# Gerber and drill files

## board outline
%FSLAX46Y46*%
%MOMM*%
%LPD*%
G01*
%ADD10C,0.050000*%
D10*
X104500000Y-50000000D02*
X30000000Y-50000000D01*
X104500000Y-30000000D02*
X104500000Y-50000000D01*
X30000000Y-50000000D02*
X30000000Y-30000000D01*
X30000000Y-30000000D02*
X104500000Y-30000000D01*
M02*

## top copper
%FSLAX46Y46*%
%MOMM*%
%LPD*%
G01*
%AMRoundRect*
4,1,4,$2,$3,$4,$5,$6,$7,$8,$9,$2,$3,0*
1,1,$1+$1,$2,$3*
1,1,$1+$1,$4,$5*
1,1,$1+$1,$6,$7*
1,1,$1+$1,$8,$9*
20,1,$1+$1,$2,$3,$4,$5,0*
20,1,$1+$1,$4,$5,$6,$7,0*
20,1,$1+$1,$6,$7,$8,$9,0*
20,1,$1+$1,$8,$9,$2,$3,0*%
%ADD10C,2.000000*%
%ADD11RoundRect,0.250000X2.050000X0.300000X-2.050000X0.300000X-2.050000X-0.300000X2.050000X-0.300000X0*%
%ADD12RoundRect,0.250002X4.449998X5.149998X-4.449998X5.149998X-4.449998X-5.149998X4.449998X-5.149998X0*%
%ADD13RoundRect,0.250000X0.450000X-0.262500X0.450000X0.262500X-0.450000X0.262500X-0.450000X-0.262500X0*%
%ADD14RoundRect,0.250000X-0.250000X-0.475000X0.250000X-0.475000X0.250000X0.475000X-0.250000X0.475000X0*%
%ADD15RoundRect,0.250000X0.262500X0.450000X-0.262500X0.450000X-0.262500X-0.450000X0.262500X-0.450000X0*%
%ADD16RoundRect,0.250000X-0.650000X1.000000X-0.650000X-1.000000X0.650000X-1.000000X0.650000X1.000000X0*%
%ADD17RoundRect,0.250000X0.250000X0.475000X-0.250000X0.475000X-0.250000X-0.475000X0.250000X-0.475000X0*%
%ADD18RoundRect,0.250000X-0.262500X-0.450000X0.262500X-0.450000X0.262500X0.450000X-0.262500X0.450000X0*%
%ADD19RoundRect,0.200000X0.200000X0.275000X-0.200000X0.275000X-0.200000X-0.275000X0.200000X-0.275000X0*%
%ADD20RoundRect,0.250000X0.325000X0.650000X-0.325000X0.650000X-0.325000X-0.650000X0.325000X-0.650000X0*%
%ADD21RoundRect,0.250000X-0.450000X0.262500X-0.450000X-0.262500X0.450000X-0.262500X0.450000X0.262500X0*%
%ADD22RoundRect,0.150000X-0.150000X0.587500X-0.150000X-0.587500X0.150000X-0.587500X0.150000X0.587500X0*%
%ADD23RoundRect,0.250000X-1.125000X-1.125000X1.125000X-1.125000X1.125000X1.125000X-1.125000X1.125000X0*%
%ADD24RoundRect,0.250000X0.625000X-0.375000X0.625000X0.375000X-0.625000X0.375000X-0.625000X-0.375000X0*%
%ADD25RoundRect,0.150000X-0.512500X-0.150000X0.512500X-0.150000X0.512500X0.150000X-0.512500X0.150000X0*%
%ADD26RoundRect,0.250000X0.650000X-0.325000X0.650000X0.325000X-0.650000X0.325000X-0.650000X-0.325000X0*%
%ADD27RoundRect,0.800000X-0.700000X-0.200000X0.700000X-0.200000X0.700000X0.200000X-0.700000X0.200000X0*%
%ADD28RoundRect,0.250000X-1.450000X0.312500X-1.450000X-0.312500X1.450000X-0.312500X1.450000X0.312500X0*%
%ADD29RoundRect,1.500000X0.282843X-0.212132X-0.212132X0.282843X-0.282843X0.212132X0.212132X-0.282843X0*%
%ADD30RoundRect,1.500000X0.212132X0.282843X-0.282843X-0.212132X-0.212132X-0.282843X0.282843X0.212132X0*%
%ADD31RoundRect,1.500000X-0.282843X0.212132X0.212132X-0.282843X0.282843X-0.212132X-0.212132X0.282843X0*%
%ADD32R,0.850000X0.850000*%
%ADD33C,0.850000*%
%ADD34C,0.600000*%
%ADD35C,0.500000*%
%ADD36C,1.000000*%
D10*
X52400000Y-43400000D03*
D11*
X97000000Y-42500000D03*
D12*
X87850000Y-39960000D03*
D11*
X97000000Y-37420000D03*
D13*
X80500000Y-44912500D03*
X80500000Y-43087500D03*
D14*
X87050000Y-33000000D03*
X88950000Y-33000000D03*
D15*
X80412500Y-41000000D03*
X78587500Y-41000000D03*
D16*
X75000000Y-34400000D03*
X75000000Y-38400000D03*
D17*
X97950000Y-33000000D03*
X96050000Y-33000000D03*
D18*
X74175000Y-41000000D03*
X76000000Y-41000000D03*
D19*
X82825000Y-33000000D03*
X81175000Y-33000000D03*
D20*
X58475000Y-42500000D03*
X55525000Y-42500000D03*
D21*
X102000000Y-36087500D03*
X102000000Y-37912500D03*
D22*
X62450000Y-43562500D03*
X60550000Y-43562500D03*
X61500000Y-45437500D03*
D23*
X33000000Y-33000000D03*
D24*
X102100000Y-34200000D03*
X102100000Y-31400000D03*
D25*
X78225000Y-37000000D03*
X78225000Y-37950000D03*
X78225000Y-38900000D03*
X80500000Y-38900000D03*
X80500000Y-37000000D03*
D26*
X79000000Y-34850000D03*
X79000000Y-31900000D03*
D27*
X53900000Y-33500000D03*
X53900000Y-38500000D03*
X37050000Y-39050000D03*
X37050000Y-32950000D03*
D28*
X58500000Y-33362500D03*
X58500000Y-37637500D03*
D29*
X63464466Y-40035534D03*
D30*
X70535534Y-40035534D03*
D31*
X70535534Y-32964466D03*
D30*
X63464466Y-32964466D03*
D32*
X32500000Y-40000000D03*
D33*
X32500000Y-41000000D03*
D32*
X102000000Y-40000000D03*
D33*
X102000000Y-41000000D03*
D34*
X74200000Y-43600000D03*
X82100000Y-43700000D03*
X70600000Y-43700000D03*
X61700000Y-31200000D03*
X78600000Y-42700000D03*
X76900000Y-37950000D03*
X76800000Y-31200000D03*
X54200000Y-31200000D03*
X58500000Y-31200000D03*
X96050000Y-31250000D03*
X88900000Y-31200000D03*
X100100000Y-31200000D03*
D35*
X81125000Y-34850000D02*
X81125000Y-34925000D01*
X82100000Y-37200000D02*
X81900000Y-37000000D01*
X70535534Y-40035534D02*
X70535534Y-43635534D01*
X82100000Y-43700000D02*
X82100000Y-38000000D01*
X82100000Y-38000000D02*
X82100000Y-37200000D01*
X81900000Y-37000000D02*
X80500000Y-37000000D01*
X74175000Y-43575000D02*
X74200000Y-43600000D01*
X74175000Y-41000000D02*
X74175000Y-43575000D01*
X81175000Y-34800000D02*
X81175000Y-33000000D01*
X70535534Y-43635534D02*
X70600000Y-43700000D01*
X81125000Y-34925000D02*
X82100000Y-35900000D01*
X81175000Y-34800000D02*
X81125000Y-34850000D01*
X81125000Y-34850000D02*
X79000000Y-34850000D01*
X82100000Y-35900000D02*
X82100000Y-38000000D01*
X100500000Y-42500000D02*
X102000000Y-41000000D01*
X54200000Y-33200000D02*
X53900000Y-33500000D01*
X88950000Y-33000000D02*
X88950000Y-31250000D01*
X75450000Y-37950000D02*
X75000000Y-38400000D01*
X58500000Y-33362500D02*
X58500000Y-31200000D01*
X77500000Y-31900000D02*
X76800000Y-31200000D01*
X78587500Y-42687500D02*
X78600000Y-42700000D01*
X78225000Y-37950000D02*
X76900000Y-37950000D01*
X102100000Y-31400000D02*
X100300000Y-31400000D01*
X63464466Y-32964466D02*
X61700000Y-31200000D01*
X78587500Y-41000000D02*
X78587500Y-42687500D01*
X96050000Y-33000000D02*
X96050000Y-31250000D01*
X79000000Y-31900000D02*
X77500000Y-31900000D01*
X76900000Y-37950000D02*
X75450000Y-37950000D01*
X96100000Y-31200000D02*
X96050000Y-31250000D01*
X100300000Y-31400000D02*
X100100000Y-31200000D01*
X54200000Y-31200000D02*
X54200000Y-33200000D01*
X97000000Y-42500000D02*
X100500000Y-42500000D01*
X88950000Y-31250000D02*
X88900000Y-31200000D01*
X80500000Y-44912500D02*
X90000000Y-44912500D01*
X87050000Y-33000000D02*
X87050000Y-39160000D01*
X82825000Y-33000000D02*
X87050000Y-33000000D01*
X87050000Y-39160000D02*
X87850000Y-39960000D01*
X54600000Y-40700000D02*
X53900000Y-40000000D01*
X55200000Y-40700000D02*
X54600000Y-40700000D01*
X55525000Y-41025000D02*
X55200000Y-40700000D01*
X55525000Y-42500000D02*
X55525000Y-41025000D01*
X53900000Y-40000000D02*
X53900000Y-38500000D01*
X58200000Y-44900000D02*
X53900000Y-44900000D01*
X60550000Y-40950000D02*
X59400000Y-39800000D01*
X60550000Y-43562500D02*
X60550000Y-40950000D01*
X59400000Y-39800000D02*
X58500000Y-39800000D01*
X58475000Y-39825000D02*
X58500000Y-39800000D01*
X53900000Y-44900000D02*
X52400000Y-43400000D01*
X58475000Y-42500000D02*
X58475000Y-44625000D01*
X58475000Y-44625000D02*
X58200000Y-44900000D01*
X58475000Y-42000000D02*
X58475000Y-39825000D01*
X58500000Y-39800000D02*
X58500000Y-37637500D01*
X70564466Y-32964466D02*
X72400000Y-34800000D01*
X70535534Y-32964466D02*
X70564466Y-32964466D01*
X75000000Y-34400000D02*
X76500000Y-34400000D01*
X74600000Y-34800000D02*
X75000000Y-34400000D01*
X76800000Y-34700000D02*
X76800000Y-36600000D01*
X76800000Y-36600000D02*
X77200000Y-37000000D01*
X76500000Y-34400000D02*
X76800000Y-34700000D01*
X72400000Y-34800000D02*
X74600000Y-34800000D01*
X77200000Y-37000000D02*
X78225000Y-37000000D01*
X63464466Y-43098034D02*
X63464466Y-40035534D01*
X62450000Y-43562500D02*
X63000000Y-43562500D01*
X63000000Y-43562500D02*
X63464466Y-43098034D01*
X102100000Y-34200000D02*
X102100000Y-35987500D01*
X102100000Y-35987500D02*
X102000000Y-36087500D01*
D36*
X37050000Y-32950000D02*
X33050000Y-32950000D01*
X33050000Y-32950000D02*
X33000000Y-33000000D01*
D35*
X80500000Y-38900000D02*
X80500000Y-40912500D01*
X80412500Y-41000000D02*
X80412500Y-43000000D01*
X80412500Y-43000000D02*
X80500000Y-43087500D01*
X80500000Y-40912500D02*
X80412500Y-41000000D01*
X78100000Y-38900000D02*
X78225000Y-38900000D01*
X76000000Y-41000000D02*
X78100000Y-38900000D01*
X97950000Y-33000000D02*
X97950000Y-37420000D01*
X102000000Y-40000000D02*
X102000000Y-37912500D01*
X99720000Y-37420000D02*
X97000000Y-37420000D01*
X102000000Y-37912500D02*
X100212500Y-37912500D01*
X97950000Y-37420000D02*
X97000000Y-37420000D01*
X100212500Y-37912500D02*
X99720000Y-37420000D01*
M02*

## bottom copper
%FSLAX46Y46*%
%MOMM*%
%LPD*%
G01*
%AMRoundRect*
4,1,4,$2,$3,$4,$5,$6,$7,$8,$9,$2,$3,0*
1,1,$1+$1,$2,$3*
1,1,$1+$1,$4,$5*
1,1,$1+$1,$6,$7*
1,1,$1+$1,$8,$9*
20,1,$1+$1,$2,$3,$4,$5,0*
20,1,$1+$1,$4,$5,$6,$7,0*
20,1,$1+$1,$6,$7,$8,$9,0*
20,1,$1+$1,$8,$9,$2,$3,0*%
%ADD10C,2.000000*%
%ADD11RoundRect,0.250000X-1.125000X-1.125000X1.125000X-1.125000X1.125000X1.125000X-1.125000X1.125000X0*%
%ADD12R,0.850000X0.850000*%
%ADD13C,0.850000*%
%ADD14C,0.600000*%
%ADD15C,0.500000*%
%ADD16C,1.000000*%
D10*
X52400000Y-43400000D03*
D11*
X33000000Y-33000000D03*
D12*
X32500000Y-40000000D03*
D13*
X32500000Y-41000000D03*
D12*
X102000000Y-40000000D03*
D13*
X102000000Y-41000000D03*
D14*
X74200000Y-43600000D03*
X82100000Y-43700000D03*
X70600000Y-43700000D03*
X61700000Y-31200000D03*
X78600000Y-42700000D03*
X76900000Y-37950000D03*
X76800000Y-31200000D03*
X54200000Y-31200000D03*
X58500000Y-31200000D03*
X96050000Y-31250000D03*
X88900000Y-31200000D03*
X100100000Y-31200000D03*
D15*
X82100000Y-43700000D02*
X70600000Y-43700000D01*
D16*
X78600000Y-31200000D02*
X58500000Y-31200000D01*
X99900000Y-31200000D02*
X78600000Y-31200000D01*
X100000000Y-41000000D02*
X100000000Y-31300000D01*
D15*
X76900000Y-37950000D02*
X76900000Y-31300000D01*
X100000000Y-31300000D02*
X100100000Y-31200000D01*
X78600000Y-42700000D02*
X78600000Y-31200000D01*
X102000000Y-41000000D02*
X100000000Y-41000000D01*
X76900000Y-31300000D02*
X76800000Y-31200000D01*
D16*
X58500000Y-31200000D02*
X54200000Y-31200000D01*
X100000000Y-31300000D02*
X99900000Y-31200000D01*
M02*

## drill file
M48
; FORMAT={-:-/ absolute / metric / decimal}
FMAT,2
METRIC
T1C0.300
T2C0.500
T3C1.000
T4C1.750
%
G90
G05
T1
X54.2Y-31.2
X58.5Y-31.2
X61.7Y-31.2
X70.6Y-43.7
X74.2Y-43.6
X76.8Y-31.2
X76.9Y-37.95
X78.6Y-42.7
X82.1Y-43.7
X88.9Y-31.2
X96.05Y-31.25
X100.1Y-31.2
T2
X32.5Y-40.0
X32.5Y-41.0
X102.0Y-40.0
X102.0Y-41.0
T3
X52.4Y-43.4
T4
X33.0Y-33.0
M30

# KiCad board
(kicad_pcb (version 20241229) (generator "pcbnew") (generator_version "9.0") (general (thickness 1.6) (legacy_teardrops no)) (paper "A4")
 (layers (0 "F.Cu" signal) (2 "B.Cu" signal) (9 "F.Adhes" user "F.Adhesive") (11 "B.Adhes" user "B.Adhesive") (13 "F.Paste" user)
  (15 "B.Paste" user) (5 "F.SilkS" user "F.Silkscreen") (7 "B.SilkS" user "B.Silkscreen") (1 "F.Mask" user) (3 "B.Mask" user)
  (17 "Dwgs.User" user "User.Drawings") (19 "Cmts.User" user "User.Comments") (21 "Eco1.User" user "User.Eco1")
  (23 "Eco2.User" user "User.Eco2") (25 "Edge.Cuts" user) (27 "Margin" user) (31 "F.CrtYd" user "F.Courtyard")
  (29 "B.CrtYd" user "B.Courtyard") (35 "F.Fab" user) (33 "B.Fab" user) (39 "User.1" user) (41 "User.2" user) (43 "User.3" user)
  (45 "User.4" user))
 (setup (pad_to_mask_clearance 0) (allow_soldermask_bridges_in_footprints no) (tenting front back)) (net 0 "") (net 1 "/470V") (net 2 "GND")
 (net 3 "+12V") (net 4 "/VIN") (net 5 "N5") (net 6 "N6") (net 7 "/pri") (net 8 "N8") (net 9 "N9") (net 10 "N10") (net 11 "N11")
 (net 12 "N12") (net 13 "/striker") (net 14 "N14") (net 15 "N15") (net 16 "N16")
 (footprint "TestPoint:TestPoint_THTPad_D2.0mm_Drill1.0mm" (layer "F.Cu") (at 52.4 43.4)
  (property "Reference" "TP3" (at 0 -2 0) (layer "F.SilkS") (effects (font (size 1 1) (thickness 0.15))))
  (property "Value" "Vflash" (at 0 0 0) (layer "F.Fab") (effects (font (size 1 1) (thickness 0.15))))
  (pad "1" thru_hole circle (at 0 0) (size 2 2) (drill 1) (layers "*.Cu" "*.Mask") (remove_unused_layers no) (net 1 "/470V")))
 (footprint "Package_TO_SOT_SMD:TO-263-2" (layer "F.Cu") (at 89.35 39.96 180)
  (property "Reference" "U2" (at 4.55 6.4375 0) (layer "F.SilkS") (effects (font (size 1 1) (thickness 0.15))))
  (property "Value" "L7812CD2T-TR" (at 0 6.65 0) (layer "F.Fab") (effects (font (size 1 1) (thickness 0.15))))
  (pad "" smd roundrect (at -0.925 -2.775 180) (size 4.55 5.25) (layers "F.Paste") (roundrect_rratio 0.054945))
  (pad "" smd roundrect (at -0.925 2.775 180) (size 4.55 5.25) (layers "F.Paste") (roundrect_rratio 0.054945))
  (pad "" smd roundrect (at 3.925 -2.775 180) (size 4.55 5.25) (layers "F.Paste") (roundrect_rratio 0.054945))
  (pad "" smd roundrect (at 3.925 2.775 180) (size 4.55 5.25) (layers "F.Paste") (roundrect_rratio 0.054945))
  (pad "1" smd roundrect (at -7.65 -2.54 180) (size 4.6 1.1) (layers "F.Cu" "F.Mask" "F.Paste") (roundrect_rratio 0.227273) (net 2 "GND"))
  (pad "2" smd roundrect (at 1.5 0 180) (size 9.4 10.8) (layers "F.Cu" "F.Mask") (roundrect_rratio 0.026596) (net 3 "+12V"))
  (pad "3" smd roundrect (at -7.65 2.54 180) (size 4.6 1.1) (layers "F.Cu" "F.Mask" "F.Paste") (roundrect_rratio 0.227273) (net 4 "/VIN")))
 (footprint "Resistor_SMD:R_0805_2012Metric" (layer "F.Cu") (at 80.5 44 90)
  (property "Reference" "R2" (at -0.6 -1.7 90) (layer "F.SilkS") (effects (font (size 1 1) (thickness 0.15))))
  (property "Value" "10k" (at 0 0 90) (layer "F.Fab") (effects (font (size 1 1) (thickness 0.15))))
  (pad "1" smd roundrect (at -0.9125 0 90) (size 1.025 1.4) (layers "F.Cu" "F.Mask" "F.Paste") (roundrect_rratio 0.243902) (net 3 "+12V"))
  (pad "2" smd roundrect (at 0.9125 0 90) (size 1.025 1.4) (layers "F.Cu" "F.Mask" "F.Paste") (roundrect_rratio 0.243902) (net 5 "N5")))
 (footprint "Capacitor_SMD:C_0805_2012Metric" (layer "F.Cu") (at 88 33)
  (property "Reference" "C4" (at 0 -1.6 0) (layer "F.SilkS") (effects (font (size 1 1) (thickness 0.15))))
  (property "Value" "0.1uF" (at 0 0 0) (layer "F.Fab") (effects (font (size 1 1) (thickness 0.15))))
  (pad "1" smd roundrect (at -0.95 0) (size 1 1.45) (layers "F.Cu" "F.Mask" "F.Paste") (roundrect_rratio 0.25) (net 3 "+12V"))
  (pad "2" smd roundrect (at 0.95 0) (size 1 1.45) (layers "F.Cu" "F.Mask" "F.Paste") (roundrect_rratio 0.25) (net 2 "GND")))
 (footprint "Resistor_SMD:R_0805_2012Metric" (layer "F.Cu") (at 79.5 41 180)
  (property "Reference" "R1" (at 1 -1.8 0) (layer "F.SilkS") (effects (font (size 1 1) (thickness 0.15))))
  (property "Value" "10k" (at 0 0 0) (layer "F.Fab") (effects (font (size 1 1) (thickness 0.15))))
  (pad "1" smd roundrect (at -0.9125 0 180) (size 1.025 1.4) (layers "F.Cu" "F.Mask" "F.Paste") (roundrect_rratio 0.243902) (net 5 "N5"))
  (pad "2" smd roundrect (at 0.9125 0 180) (size 1.025 1.4) (layers "F.Cu" "F.Mask" "F.Paste") (roundrect_rratio 0.243902) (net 2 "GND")))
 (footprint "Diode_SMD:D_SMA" (layer "F.Cu") (at 75 36.4 -90)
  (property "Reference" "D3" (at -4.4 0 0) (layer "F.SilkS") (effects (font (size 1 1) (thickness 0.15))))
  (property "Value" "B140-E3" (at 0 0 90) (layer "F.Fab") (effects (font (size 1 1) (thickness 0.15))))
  (pad "1" smd roundrect (at -2 0 270) (size 2.5 1.8) (layers "F.Cu" "F.Mask" "F.Paste") (roundrect_rratio 0.1388888889) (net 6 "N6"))
  (pad "2" smd roundrect (at 2 0 270) (size 2.5 1.8) (layers "F.Cu" "F.Mask" "F.Paste") (roundrect_rratio 0.1388888889) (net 2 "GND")))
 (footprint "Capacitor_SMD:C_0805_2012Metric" (layer "F.Cu") (at 97 33 180)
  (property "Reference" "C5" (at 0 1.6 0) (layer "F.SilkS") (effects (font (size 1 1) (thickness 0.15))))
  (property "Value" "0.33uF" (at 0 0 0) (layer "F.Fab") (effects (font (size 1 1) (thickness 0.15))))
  (pad "1" smd roundrect (at -0.95 0 180) (size 1 1.45) (layers "F.Cu" "F.Mask" "F.Paste") (roundrect_rratio 0.25) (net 4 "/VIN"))
  (pad "2" smd roundrect (at 0.95 0 180) (size 1 1.45) (layers "F.Cu" "F.Mask" "F.Paste") (roundrect_rratio 0.25) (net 2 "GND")))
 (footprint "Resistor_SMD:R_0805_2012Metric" (layer "F.Cu") (at 75.0875 41)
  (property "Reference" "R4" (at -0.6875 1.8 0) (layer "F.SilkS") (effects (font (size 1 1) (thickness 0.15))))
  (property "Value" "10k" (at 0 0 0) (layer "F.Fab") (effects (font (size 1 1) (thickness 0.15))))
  (pad "1" smd roundrect (at -0.9125 0) (size 1.025 1.4) (layers "F.Cu" "F.Mask" "F.Paste") (roundrect_rratio 0.243902) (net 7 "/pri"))
  (pad "2" smd roundrect (at 0.9125 0) (size 1.025 1.4) (layers "F.Cu" "F.Mask" "F.Paste") (roundrect_rratio 0.243902) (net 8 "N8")))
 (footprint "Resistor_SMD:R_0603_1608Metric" (layer "F.Cu") (at 82 33 180)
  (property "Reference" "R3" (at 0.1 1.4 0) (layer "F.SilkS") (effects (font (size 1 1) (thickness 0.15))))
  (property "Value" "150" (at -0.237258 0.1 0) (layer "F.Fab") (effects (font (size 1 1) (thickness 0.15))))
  (pad "1" smd roundrect (at -0.825 0 180) (size 0.8 0.95) (layers "F.Cu" "F.Mask" "F.Paste") (roundrect_rratio 0.25) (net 3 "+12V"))
  (pad "2" smd roundrect (at 0.825 0 180) (size 0.8 0.95) (layers "F.Cu" "F.Mask" "F.Paste") (roundrect_rratio 0.25) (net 7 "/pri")))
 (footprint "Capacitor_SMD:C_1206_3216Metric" (layer "F.Cu") (at 57 42.5 180)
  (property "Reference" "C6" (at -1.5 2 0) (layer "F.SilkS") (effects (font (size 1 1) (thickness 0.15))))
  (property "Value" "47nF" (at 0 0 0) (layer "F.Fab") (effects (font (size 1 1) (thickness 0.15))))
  (pad "1" smd roundrect (at -1.475 0 180) (size 1.15 1.8) (layers "F.Cu" "F.Mask" "F.Paste") (roundrect_rratio 0.217391) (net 1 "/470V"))
  (pad "2" smd roundrect (at 1.475 0 180) (size 1.15 1.8) (layers "F.Cu" "F.Mask" "F.Paste") (roundrect_rratio 0.217391) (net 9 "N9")))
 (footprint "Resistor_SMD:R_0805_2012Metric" (layer "F.Cu") (at 102 37 -90)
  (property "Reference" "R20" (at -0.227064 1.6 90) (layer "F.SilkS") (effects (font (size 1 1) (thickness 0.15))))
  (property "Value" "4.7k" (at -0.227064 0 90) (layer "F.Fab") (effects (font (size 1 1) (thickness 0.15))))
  (pad "1" smd roundrect (at -0.9125 0 270) (size 1.025 1.4) (layers "F.Cu" "F.Mask" "F.Paste") (roundrect_rratio 0.243902) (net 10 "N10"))
  (pad "2" smd roundrect (at 0.9125 0 270) (size 1.025 1.4) (layers "F.Cu" "F.Mask" "F.Paste") (roundrect_rratio 0.243902) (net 4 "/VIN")))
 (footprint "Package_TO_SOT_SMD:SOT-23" (layer "F.Cu") (at 61.5 44.5 -90)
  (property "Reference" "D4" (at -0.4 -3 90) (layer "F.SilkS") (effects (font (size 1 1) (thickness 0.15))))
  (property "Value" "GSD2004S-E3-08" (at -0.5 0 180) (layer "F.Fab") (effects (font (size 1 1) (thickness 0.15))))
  (pad "1" smd roundrect (at -0.9375 -0.95 270) (size 1.475 0.6) (layers "F.Cu" "F.Mask" "F.Paste") (roundrect_rratio 0.25) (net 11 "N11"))
  (pad "2" smd roundrect (at -0.9375 0.95 270) (size 1.475 0.6) (layers "F.Cu" "F.Mask" "F.Paste") (roundrect_rratio 0.25) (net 1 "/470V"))
  (pad "3" smd roundrect (at 0.9375 0 270) (size 1.475 0.6) (layers "F.Cu" "F.Mask" "F.Paste") (roundrect_rratio 0.25) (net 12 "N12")))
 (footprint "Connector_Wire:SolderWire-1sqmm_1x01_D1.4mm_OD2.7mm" (layer "F.Cu") (at 33 33)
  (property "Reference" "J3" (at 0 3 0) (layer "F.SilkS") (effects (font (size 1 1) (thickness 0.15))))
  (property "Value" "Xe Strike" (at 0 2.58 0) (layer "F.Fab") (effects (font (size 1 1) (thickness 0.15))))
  (pad "1" thru_hole roundrect (at 0 0) (size 2.75 2.75) (drill 1.75) (layers "*.Cu" "*.Mask") (remove_unused_layers no)
   (roundrect_rratio 0.090909) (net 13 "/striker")))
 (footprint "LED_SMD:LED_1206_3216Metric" (layer "F.Cu") (at 102.1 32.8 90)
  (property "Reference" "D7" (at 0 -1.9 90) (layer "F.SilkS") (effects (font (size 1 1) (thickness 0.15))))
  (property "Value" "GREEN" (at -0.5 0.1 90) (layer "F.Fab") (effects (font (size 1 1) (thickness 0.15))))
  (pad "1" smd roundrect (at -1.4 0 90) (size 1.25 1.75) (layers "F.Cu" "F.Mask" "F.Paste") (roundrect_rratio 0.2) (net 10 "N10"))
  (pad "2" smd roundrect (at 1.4 0 90) (size 1.25 1.75) (layers "F.Cu" "F.Mask" "F.Paste") (roundrect_rratio 0.2) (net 2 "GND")))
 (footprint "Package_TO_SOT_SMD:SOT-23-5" (layer "F.Cu") (at 79.3625 37.95)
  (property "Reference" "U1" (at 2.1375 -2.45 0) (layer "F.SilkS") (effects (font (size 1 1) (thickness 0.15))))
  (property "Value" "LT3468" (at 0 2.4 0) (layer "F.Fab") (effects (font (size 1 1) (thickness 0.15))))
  (pad "1" smd roundrect (at -1.1375 -0.95) (size 1.325 0.6) (layers "F.Cu" "F.Mask" "F.Paste") (roundrect_rratio 0.25) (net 6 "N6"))
  (pad "2" smd roundrect (at -1.1375 0) (size 1.325 0.6) (layers "F.Cu" "F.Mask" "F.Paste") (roundrect_rratio 0.25) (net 2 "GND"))
  (pad "3" smd roundrect (at -1.1375 0.95) (size 1.325 0.6) (layers "F.Cu" "F.Mask" "F.Paste") (roundrect_rratio 0.25) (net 8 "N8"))
  (pad "4" smd roundrect (at 1.1375 0.95) (size 1.325 0.6) (layers "F.Cu" "F.Mask" "F.Paste") (roundrect_rratio 0.25) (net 5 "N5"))
  (pad "5" smd roundrect (at 1.1375 -0.95) (size 1.325 0.6) (layers "F.Cu" "F.Mask" "F.Paste") (roundrect_rratio 0.25) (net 7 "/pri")))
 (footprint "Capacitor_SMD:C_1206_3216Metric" (layer "F.Cu") (at 79 33.375 90)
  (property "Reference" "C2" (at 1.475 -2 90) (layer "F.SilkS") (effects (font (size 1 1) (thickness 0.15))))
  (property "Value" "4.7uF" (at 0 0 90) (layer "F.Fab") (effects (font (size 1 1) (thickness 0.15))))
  (pad "1" smd roundrect (at -1.475 0 90) (size 1.15 1.8) (layers "F.Cu" "F.Mask" "F.Paste") (roundrect_rratio 0.217391) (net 7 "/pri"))
  (pad "2" smd roundrect (at 1.475 0 90) (size 1.15 1.8) (layers "F.Cu" "F.Mask" "F.Paste") (roundrect_rratio 0.217391) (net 2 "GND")))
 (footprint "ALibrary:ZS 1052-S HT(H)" (layer "F.Cu") (at 45.5 36 180)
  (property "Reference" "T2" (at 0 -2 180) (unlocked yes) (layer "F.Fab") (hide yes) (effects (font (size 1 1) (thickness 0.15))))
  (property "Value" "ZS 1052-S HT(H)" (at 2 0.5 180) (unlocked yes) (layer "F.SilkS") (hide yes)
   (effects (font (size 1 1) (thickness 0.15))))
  (pad "1" smd roundrect (at -8.4 2.5) (size 3 2) (layers "F.Cu" "F.Mask" "F.Paste") (roundrect_rratio 0.4) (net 2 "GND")
   (thermal_bridge_angle 45))
  (pad "2" smd roundrect (at -8.4 -2.5) (size 3 2) (layers "F.Cu" "F.Mask" "F.Paste") (roundrect_rratio 0.4) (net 9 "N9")
   (thermal_bridge_angle 45))
  (pad "3" smd roundrect (at 8.45 -3.05) (size 3 2) (layers "F.Cu" "F.Mask" "F.Paste") (roundrect_rratio 0.4) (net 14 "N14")
   (thermal_bridge_angle 45))
  (pad "4" smd roundrect (at 8.45 3.05) (size 3 2) (layers "F.Cu" "F.Mask" "F.Paste") (roundrect_rratio 0.4) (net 13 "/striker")
   (thermal_bridge_angle 45)))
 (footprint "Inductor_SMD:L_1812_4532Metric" (layer "F.Cu") (at 58.5 35.5 -90)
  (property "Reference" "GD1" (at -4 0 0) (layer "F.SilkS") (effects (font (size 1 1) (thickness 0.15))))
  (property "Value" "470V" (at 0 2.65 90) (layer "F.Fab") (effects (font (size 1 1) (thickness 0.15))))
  (pad "1" smd roundrect (at -2.1375 0 270) (size 1.125 3.4) (layers "F.Cu" "F.Mask" "F.Paste") (roundrect_rratio 0.222222) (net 2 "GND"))
  (pad "2" smd roundrect (at 2.1375 0 270) (size 1.125 3.4) (layers "F.Cu" "F.Mask" "F.Paste") (roundrect_rratio 0.222222) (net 1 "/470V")))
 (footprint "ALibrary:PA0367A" (layer "F.Cu") (at 67 36.5 135)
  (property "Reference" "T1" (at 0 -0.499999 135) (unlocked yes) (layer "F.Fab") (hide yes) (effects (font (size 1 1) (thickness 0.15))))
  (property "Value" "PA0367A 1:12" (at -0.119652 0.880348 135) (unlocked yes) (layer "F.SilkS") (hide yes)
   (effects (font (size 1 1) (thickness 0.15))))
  (pad "1" smd roundrect (at 0 -5 135) (size 3.7 3.1) (layers "F.Cu" "F.Mask" "F.Paste") (roundrect_rratio 0.4838709677) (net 11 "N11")
   (thermal_bridge_angle 45))
  (pad "2" smd roundrect (at -5 0 225) (size 3.7 3.1) (layers "F.Cu" "F.Mask" "F.Paste") (roundrect_rratio 0.4838709677) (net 7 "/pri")
   (thermal_bridge_angle 45))
  (pad "3" smd roundrect (at 0 5 315) (size 3.7 3.1) (layers "F.Cu" "F.Mask" "F.Paste") (roundrect_rratio 0.4838709677) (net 6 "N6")
   (thermal_bridge_angle 45))
  (pad "4" smd roundrect (at 5 0 225) (size 3.7 3.1) (layers "F.Cu" "F.Mask" "F.Paste") (roundrect_rratio 0.4838709677) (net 2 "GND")
   (thermal_bridge_angle 45)))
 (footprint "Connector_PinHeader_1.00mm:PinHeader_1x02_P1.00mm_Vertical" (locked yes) (layer "B.Cu") (at 32.5 40 180)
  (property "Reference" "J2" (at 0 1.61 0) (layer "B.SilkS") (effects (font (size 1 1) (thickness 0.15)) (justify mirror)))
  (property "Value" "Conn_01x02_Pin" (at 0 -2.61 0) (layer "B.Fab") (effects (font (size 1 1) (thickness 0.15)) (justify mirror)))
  (pad "1" thru_hole rect (at 0 0 180) (size 0.85 0.85) (drill 0.5) (layers "*.Cu" "*.Mask") (remove_unused_layers no) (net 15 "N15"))
  (pad "2" thru_hole circle (at 0 -1 180) (size 0.85 0.85) (drill 0.5) (layers "*.Cu" "*.Mask") (remove_unused_layers no) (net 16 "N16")))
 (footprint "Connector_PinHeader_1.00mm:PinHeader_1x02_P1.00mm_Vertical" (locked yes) (layer "B.Cu") (at 102 40 180)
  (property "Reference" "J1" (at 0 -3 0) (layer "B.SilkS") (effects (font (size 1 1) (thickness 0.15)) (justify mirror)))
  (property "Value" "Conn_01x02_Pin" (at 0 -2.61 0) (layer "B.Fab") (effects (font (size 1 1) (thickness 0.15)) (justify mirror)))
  (pad "1" thru_hole rect (at 0 0 180) (size 0.85 0.85) (drill 0.5) (layers "*.Cu" "*.Mask") (remove_unused_layers no) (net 4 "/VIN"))
  (pad "2" thru_hole circle (at 0 -1 180) (size 0.85 0.85) (drill 0.5) (layers "*.Cu" "*.Mask") (remove_unused_layers no) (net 2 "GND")))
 (gr_line (start 104.5 50) (end 30 50) (stroke (width 0.05) (type default)) (layer "Edge.Cuts"))
 (gr_line (start 104.5 30) (end 104.5 50) (stroke (width 0.05) (type default)) (layer "Edge.Cuts"))
 (gr_line (start 30 50) (end 30 30) (stroke (width 0.05) (type default)) (layer "Edge.Cuts"))
 (gr_line (start 30 30) (end 104.5 30) (stroke (width 0.05) (type default)) (layer "Edge.Cuts"))
 (segment (start 81.125 34.85) (end 81.125 34.925) (width 0.5) (layer "F.Cu") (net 7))
 (segment (start 82.1 37.2) (end 81.9 37) (width 0.5) (layer "F.Cu") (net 7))
 (segment (start 70.535534 40.035534) (end 70.535534 43.635534) (width 0.5) (layer "F.Cu") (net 7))
 (segment (start 82.1 43.7) (end 82.1 38) (width 0.5) (layer "F.Cu") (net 7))
 (segment (start 82.1 38) (end 82.1 37.2) (width 0.5) (layer "F.Cu") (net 7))
 (segment (start 81.9 37) (end 80.5 37) (width 0.5) (layer "F.Cu") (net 7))
 (segment (start 74.175 43.575) (end 74.2 43.6) (width 0.5) (layer "F.Cu") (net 7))
 (segment (start 74.175 41) (end 74.175 43.575) (width 0.5) (layer "F.Cu") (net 7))
 (segment (start 81.175 34.8) (end 81.175 33) (width 0.5) (layer "F.Cu") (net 7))
 (segment (start 70.535534 43.635534) (end 70.6 43.7) (width 0.5) (layer "F.Cu") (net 7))
 (segment (start 81.125 34.925) (end 82.1 35.9) (width 0.5) (layer "F.Cu") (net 7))
 (segment (start 81.175 34.8) (end 81.125 34.85) (width 0.5) (layer "F.Cu") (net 7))
 (segment (start 81.125 34.85) (end 79 34.85) (width 0.5) (layer "F.Cu") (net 7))
 (segment (start 82.1 35.9) (end 82.1 38) (width 0.5) (layer "F.Cu") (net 7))
 (via (at 74.2 43.6) (size 0.6) (drill 0.3) (layers "F.Cu" "B.Cu") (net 7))
 (via (at 82.1 43.7) (size 0.6) (drill 0.3) (layers "F.Cu" "B.Cu") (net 7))
 (via (at 70.6 43.7) (size 0.6) (drill 0.3) (layers "F.Cu" "B.Cu") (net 7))
 (segment (start 82.1 43.7) (end 70.6 43.7) (width 0.5) (layer "B.Cu") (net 7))
 (segment (start 100.5 42.5) (end 102 41) (width 0.5) (layer "F.Cu") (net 2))
 (segment (start 54.2 33.2) (end 53.9 33.5) (width 0.5) (layer "F.Cu") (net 2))
 (segment (start 88.95 33) (end 88.95 31.25) (width 0.5) (layer "F.Cu") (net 2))
 (segment (start 75.45 37.95) (end 75 38.4) (width 0.5) (layer "F.Cu") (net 2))
 (segment (start 58.5 33.3625) (end 58.5 31.2) (width 0.5) (layer "F.Cu") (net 2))
 (segment (start 77.5 31.9) (end 76.8 31.2) (width 0.5) (layer "F.Cu") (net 2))
 (segment (start 78.5875 42.6875) (end 78.6 42.7) (width 0.5) (layer "F.Cu") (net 2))
 (segment (start 78.225 37.95) (end 76.9 37.95) (width 0.5) (layer "F.Cu") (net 2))
 (segment (start 102.1 31.4) (end 100.3 31.4) (width 0.5) (layer "F.Cu") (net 2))
 (segment (start 63.464466 32.964466) (end 61.7 31.2) (width 0.5) (layer "F.Cu") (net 2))
 (segment (start 78.5875 41) (end 78.5875 42.6875) (width 0.5) (layer "F.Cu") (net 2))
 (segment (start 96.05 33) (end 96.05 31.25) (width 0.5) (layer "F.Cu") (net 2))
 (segment (start 79 31.9) (end 77.5 31.9) (width 0.5) (layer "F.Cu") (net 2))
 (segment (start 76.9 37.95) (end 75.45 37.95) (width 0.5) (layer "F.Cu") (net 2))
 (segment (start 96.1 31.2) (end 96.05 31.25) (width 0.5) (layer "F.Cu") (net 2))
 (segment (start 100.3 31.4) (end 100.1 31.2) (width 0.5) (layer "F.Cu") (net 2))
 (segment (start 54.2 31.2) (end 54.2 33.2) (width 0.5) (layer "F.Cu") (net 2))
 (segment (start 97 42.5) (end 100.5 42.5) (width 0.5) (layer "F.Cu") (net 2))
 (segment (start 88.95 31.25) (end 88.9 31.2) (width 0.5) (layer "F.Cu") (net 2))
 (via (at 61.7 31.2) (size 0.6) (drill 0.3) (layers "F.Cu" "B.Cu") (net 2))
 (via (at 78.6 42.7) (size 0.6) (drill 0.3) (layers "F.Cu" "B.Cu") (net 2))
 (via (at 76.9 37.95) (size 0.6) (drill 0.3) (layers "F.Cu" "B.Cu") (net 2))
 (via (at 76.8 31.2) (size 0.6) (drill 0.3) (layers "F.Cu" "B.Cu") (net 2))
 (via (at 54.2 31.2) (size 0.6) (drill 0.3) (layers "F.Cu" "B.Cu") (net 2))
 (via (at 58.5 31.2) (size 0.6) (drill 0.3) (layers "F.Cu" "B.Cu") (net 2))
 (via (at 96.05 31.25) (size 0.6) (drill 0.3) (layers "F.Cu" "B.Cu") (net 2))
 (via (at 88.9 31.2) (size 0.6) (drill 0.3) (layers "F.Cu" "B.Cu") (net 2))
 (via (at 100.1 31.2) (size 0.6) (drill 0.3) (layers "F.Cu" "B.Cu") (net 2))
 (segment (start 78.6 31.2) (end 58.5 31.2) (width 1) (layer "B.Cu") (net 2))
 (segment (start 99.9 31.2) (end 78.6 31.2) (width 1) (layer "B.Cu") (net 2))
 (segment (start 100 41) (end 100 31.3) (width 1) (layer "B.Cu") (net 2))
 (segment (start 76.9 37.95) (end 76.9 31.3) (width 0.5) (layer "B.Cu") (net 2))
 (segment (start 100 31.3) (end 100.1 31.2) (width 0.5) (layer "B.Cu") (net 2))
 (segment (start 78.6 42.7) (end 78.6 31.2) (width 0.5) (layer "B.Cu") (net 2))
 (segment (start 102 41) (end 100 41) (width 0.5) (layer "B.Cu") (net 2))
 (segment (start 76.9 31.3) (end 76.8 31.2) (width 0.5) (layer "B.Cu") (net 2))
 (segment (start 58.5 31.2) (end 54.2 31.2) (width 1) (layer "B.Cu") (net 2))
 (segment (start 100 31.3) (end 99.9 31.2) (width 1) (layer "B.Cu") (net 2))
 (segment (start 80.5 44.9125) (end 90 44.9125) (width 0.5) (layer "F.Cu") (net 3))
 (segment (start 87.05 33) (end 87.05 39.16) (width 0.5) (layer "F.Cu") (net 3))
 (segment (start 82.825 33) (end 87.05 33) (width 0.5) (layer "F.Cu") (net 3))
 (segment (start 87.05 39.16) (end 87.85 39.96) (width 0.5) (layer "F.Cu") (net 3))
 (segment (start 54.6 40.7) (end 53.9 40) (width 0.5) (layer "F.Cu") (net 9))
 (segment (start 55.2 40.7) (end 54.6 40.7) (width 0.5) (layer "F.Cu") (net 9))
 (segment (start 55.525 41.025) (end 55.2 40.7) (width 0.5) (layer "F.Cu") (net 9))
 (segment (start 55.525 42.5) (end 55.525 41.025) (width 0.5) (layer "F.Cu") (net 9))
 (segment (start 53.9 40) (end 53.9 38.5) (width 0.5) (layer "F.Cu") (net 9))
 (segment (start 58.2 44.9) (end 53.9 44.9) (width 0.5) (layer "F.Cu") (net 1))
 (segment (start 60.55 40.95) (end 59.4 39.8) (width 0.5) (layer "F.Cu") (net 1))
 (segment (start 60.55 43.5625) (end 60.55 40.95) (width 0.5) (layer "F.Cu") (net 1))
 (segment (start 59.4 39.8) (end 58.5 39.8) (width 0.5) (layer "F.Cu") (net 1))
 (segment (start 58.475 39.825) (end 58.5 39.8) (width 0.5) (layer "F.Cu") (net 1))
 (segment (start 53.9 44.9) (end 52.4 43.4) (width 0.5) (layer "F.Cu") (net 1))
 (segment (start 58.475 42.5) (end 58.475 44.625) (width 0.5) (layer "F.Cu") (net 1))
 (segment (start 58.475 44.625) (end 58.2 44.9) (width 0.5) (layer "F.Cu") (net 1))
 (segment (start 58.475 42) (end 58.475 39.825) (width 0.5) (layer "F.Cu") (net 1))
 (segment (start 58.5 39.8) (end 58.5 37.6375) (width 0.5) (layer "F.Cu") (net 1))
 (segment (start 70.564466 32.964466) (end 72.4 34.8) (width 0.5) (layer "F.Cu") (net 6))
 (segment (start 70.535534 32.964466) (end 70.564466 32.964466) (width 0.5) (layer "F.Cu") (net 6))
 (segment (start 75 34.4) (end 76.5 34.4) (width 0.5) (layer "F.Cu") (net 6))
 (segment (start 74.6 34.8) (end 75 34.4) (width 0.5) (layer "F.Cu") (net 6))
 (segment (start 76.8 34.7) (end 76.8 36.6) (width 0.5) (layer "F.Cu") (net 6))
 (segment (start 76.8 36.6) (end 77.2 37) (width 0.5) (layer "F.Cu") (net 6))
 (segment (start 76.5 34.4) (end 76.8 34.7) (width 0.5) (layer "F.Cu") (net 6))
 (segment (start 72.4 34.8) (end 74.6 34.8) (width 0.5) (layer "F.Cu") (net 6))
 (segment (start 77.2 37) (end 78.225 37) (width 0.5) (layer "F.Cu") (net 6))
 (segment (start 63.464466 43.098034) (end 63.464466 40.035534) (width 0.5) (layer "F.Cu") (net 11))
 (segment (start 62.45 43.5625) (end 63 43.5625) (width 0.5) (layer "F.Cu") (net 11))
 (segment (start 63 43.5625) (end 63.464466 43.098034) (width 0.5) (layer "F.Cu") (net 11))
 (segment (start 102.1 34.2) (end 102.1 35.9875) (width 0.5) (layer "F.Cu") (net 10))
 (segment (start 102.1 35.9875) (end 102 36.0875) (width 0.5) (layer "F.Cu") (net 10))
 (segment (start 37.05 32.95) (end 33.05 32.95) (width 1) (layer "F.Cu") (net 13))
 (segment (start 33.05 32.95) (end 33 33) (width 1) (layer "F.Cu") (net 13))
 (segment (start 80.5 38.9) (end 80.5 40.9125) (width 0.5) (layer "F.Cu") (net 5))
 (segment (start 80.4125 41) (end 80.4125 43) (width 0.5) (layer "F.Cu") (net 5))
 (segment (start 80.4125 43) (end 80.5 43.0875) (width 0.5) (layer "F.Cu") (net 5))
 (segment (start 80.5 40.9125) (end 80.4125 41) (width 0.5) (layer "F.Cu") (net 5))
 (segment (start 78.1 38.9) (end 78.225 38.9) (width 0.5) (layer "F.Cu") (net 8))
 (segment (start 76 41) (end 78.1 38.9) (width 0.5) (layer "F.Cu") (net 8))
 (segment (start 97.95 33) (end 97.95 37.42) (width 0.5) (layer "F.Cu") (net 4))
 (segment (start 102 40) (end 102 37.9125) (width 0.5) (layer "F.Cu") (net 4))
 (segment (start 99.72 37.42) (end 97 37.42) (width 0.5) (layer "F.Cu") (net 4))
 (segment (start 102 37.9125) (end 100.2125 37.9125) (width 0.5) (layer "F.Cu") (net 4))
 (segment (start 97.95 37.42) (end 97 37.42) (width 0.5) (layer "F.Cu") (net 4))
 (segment (start 100.2125 37.9125) (end 99.72 37.42) (width 0.5) (layer "F.Cu") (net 4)))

